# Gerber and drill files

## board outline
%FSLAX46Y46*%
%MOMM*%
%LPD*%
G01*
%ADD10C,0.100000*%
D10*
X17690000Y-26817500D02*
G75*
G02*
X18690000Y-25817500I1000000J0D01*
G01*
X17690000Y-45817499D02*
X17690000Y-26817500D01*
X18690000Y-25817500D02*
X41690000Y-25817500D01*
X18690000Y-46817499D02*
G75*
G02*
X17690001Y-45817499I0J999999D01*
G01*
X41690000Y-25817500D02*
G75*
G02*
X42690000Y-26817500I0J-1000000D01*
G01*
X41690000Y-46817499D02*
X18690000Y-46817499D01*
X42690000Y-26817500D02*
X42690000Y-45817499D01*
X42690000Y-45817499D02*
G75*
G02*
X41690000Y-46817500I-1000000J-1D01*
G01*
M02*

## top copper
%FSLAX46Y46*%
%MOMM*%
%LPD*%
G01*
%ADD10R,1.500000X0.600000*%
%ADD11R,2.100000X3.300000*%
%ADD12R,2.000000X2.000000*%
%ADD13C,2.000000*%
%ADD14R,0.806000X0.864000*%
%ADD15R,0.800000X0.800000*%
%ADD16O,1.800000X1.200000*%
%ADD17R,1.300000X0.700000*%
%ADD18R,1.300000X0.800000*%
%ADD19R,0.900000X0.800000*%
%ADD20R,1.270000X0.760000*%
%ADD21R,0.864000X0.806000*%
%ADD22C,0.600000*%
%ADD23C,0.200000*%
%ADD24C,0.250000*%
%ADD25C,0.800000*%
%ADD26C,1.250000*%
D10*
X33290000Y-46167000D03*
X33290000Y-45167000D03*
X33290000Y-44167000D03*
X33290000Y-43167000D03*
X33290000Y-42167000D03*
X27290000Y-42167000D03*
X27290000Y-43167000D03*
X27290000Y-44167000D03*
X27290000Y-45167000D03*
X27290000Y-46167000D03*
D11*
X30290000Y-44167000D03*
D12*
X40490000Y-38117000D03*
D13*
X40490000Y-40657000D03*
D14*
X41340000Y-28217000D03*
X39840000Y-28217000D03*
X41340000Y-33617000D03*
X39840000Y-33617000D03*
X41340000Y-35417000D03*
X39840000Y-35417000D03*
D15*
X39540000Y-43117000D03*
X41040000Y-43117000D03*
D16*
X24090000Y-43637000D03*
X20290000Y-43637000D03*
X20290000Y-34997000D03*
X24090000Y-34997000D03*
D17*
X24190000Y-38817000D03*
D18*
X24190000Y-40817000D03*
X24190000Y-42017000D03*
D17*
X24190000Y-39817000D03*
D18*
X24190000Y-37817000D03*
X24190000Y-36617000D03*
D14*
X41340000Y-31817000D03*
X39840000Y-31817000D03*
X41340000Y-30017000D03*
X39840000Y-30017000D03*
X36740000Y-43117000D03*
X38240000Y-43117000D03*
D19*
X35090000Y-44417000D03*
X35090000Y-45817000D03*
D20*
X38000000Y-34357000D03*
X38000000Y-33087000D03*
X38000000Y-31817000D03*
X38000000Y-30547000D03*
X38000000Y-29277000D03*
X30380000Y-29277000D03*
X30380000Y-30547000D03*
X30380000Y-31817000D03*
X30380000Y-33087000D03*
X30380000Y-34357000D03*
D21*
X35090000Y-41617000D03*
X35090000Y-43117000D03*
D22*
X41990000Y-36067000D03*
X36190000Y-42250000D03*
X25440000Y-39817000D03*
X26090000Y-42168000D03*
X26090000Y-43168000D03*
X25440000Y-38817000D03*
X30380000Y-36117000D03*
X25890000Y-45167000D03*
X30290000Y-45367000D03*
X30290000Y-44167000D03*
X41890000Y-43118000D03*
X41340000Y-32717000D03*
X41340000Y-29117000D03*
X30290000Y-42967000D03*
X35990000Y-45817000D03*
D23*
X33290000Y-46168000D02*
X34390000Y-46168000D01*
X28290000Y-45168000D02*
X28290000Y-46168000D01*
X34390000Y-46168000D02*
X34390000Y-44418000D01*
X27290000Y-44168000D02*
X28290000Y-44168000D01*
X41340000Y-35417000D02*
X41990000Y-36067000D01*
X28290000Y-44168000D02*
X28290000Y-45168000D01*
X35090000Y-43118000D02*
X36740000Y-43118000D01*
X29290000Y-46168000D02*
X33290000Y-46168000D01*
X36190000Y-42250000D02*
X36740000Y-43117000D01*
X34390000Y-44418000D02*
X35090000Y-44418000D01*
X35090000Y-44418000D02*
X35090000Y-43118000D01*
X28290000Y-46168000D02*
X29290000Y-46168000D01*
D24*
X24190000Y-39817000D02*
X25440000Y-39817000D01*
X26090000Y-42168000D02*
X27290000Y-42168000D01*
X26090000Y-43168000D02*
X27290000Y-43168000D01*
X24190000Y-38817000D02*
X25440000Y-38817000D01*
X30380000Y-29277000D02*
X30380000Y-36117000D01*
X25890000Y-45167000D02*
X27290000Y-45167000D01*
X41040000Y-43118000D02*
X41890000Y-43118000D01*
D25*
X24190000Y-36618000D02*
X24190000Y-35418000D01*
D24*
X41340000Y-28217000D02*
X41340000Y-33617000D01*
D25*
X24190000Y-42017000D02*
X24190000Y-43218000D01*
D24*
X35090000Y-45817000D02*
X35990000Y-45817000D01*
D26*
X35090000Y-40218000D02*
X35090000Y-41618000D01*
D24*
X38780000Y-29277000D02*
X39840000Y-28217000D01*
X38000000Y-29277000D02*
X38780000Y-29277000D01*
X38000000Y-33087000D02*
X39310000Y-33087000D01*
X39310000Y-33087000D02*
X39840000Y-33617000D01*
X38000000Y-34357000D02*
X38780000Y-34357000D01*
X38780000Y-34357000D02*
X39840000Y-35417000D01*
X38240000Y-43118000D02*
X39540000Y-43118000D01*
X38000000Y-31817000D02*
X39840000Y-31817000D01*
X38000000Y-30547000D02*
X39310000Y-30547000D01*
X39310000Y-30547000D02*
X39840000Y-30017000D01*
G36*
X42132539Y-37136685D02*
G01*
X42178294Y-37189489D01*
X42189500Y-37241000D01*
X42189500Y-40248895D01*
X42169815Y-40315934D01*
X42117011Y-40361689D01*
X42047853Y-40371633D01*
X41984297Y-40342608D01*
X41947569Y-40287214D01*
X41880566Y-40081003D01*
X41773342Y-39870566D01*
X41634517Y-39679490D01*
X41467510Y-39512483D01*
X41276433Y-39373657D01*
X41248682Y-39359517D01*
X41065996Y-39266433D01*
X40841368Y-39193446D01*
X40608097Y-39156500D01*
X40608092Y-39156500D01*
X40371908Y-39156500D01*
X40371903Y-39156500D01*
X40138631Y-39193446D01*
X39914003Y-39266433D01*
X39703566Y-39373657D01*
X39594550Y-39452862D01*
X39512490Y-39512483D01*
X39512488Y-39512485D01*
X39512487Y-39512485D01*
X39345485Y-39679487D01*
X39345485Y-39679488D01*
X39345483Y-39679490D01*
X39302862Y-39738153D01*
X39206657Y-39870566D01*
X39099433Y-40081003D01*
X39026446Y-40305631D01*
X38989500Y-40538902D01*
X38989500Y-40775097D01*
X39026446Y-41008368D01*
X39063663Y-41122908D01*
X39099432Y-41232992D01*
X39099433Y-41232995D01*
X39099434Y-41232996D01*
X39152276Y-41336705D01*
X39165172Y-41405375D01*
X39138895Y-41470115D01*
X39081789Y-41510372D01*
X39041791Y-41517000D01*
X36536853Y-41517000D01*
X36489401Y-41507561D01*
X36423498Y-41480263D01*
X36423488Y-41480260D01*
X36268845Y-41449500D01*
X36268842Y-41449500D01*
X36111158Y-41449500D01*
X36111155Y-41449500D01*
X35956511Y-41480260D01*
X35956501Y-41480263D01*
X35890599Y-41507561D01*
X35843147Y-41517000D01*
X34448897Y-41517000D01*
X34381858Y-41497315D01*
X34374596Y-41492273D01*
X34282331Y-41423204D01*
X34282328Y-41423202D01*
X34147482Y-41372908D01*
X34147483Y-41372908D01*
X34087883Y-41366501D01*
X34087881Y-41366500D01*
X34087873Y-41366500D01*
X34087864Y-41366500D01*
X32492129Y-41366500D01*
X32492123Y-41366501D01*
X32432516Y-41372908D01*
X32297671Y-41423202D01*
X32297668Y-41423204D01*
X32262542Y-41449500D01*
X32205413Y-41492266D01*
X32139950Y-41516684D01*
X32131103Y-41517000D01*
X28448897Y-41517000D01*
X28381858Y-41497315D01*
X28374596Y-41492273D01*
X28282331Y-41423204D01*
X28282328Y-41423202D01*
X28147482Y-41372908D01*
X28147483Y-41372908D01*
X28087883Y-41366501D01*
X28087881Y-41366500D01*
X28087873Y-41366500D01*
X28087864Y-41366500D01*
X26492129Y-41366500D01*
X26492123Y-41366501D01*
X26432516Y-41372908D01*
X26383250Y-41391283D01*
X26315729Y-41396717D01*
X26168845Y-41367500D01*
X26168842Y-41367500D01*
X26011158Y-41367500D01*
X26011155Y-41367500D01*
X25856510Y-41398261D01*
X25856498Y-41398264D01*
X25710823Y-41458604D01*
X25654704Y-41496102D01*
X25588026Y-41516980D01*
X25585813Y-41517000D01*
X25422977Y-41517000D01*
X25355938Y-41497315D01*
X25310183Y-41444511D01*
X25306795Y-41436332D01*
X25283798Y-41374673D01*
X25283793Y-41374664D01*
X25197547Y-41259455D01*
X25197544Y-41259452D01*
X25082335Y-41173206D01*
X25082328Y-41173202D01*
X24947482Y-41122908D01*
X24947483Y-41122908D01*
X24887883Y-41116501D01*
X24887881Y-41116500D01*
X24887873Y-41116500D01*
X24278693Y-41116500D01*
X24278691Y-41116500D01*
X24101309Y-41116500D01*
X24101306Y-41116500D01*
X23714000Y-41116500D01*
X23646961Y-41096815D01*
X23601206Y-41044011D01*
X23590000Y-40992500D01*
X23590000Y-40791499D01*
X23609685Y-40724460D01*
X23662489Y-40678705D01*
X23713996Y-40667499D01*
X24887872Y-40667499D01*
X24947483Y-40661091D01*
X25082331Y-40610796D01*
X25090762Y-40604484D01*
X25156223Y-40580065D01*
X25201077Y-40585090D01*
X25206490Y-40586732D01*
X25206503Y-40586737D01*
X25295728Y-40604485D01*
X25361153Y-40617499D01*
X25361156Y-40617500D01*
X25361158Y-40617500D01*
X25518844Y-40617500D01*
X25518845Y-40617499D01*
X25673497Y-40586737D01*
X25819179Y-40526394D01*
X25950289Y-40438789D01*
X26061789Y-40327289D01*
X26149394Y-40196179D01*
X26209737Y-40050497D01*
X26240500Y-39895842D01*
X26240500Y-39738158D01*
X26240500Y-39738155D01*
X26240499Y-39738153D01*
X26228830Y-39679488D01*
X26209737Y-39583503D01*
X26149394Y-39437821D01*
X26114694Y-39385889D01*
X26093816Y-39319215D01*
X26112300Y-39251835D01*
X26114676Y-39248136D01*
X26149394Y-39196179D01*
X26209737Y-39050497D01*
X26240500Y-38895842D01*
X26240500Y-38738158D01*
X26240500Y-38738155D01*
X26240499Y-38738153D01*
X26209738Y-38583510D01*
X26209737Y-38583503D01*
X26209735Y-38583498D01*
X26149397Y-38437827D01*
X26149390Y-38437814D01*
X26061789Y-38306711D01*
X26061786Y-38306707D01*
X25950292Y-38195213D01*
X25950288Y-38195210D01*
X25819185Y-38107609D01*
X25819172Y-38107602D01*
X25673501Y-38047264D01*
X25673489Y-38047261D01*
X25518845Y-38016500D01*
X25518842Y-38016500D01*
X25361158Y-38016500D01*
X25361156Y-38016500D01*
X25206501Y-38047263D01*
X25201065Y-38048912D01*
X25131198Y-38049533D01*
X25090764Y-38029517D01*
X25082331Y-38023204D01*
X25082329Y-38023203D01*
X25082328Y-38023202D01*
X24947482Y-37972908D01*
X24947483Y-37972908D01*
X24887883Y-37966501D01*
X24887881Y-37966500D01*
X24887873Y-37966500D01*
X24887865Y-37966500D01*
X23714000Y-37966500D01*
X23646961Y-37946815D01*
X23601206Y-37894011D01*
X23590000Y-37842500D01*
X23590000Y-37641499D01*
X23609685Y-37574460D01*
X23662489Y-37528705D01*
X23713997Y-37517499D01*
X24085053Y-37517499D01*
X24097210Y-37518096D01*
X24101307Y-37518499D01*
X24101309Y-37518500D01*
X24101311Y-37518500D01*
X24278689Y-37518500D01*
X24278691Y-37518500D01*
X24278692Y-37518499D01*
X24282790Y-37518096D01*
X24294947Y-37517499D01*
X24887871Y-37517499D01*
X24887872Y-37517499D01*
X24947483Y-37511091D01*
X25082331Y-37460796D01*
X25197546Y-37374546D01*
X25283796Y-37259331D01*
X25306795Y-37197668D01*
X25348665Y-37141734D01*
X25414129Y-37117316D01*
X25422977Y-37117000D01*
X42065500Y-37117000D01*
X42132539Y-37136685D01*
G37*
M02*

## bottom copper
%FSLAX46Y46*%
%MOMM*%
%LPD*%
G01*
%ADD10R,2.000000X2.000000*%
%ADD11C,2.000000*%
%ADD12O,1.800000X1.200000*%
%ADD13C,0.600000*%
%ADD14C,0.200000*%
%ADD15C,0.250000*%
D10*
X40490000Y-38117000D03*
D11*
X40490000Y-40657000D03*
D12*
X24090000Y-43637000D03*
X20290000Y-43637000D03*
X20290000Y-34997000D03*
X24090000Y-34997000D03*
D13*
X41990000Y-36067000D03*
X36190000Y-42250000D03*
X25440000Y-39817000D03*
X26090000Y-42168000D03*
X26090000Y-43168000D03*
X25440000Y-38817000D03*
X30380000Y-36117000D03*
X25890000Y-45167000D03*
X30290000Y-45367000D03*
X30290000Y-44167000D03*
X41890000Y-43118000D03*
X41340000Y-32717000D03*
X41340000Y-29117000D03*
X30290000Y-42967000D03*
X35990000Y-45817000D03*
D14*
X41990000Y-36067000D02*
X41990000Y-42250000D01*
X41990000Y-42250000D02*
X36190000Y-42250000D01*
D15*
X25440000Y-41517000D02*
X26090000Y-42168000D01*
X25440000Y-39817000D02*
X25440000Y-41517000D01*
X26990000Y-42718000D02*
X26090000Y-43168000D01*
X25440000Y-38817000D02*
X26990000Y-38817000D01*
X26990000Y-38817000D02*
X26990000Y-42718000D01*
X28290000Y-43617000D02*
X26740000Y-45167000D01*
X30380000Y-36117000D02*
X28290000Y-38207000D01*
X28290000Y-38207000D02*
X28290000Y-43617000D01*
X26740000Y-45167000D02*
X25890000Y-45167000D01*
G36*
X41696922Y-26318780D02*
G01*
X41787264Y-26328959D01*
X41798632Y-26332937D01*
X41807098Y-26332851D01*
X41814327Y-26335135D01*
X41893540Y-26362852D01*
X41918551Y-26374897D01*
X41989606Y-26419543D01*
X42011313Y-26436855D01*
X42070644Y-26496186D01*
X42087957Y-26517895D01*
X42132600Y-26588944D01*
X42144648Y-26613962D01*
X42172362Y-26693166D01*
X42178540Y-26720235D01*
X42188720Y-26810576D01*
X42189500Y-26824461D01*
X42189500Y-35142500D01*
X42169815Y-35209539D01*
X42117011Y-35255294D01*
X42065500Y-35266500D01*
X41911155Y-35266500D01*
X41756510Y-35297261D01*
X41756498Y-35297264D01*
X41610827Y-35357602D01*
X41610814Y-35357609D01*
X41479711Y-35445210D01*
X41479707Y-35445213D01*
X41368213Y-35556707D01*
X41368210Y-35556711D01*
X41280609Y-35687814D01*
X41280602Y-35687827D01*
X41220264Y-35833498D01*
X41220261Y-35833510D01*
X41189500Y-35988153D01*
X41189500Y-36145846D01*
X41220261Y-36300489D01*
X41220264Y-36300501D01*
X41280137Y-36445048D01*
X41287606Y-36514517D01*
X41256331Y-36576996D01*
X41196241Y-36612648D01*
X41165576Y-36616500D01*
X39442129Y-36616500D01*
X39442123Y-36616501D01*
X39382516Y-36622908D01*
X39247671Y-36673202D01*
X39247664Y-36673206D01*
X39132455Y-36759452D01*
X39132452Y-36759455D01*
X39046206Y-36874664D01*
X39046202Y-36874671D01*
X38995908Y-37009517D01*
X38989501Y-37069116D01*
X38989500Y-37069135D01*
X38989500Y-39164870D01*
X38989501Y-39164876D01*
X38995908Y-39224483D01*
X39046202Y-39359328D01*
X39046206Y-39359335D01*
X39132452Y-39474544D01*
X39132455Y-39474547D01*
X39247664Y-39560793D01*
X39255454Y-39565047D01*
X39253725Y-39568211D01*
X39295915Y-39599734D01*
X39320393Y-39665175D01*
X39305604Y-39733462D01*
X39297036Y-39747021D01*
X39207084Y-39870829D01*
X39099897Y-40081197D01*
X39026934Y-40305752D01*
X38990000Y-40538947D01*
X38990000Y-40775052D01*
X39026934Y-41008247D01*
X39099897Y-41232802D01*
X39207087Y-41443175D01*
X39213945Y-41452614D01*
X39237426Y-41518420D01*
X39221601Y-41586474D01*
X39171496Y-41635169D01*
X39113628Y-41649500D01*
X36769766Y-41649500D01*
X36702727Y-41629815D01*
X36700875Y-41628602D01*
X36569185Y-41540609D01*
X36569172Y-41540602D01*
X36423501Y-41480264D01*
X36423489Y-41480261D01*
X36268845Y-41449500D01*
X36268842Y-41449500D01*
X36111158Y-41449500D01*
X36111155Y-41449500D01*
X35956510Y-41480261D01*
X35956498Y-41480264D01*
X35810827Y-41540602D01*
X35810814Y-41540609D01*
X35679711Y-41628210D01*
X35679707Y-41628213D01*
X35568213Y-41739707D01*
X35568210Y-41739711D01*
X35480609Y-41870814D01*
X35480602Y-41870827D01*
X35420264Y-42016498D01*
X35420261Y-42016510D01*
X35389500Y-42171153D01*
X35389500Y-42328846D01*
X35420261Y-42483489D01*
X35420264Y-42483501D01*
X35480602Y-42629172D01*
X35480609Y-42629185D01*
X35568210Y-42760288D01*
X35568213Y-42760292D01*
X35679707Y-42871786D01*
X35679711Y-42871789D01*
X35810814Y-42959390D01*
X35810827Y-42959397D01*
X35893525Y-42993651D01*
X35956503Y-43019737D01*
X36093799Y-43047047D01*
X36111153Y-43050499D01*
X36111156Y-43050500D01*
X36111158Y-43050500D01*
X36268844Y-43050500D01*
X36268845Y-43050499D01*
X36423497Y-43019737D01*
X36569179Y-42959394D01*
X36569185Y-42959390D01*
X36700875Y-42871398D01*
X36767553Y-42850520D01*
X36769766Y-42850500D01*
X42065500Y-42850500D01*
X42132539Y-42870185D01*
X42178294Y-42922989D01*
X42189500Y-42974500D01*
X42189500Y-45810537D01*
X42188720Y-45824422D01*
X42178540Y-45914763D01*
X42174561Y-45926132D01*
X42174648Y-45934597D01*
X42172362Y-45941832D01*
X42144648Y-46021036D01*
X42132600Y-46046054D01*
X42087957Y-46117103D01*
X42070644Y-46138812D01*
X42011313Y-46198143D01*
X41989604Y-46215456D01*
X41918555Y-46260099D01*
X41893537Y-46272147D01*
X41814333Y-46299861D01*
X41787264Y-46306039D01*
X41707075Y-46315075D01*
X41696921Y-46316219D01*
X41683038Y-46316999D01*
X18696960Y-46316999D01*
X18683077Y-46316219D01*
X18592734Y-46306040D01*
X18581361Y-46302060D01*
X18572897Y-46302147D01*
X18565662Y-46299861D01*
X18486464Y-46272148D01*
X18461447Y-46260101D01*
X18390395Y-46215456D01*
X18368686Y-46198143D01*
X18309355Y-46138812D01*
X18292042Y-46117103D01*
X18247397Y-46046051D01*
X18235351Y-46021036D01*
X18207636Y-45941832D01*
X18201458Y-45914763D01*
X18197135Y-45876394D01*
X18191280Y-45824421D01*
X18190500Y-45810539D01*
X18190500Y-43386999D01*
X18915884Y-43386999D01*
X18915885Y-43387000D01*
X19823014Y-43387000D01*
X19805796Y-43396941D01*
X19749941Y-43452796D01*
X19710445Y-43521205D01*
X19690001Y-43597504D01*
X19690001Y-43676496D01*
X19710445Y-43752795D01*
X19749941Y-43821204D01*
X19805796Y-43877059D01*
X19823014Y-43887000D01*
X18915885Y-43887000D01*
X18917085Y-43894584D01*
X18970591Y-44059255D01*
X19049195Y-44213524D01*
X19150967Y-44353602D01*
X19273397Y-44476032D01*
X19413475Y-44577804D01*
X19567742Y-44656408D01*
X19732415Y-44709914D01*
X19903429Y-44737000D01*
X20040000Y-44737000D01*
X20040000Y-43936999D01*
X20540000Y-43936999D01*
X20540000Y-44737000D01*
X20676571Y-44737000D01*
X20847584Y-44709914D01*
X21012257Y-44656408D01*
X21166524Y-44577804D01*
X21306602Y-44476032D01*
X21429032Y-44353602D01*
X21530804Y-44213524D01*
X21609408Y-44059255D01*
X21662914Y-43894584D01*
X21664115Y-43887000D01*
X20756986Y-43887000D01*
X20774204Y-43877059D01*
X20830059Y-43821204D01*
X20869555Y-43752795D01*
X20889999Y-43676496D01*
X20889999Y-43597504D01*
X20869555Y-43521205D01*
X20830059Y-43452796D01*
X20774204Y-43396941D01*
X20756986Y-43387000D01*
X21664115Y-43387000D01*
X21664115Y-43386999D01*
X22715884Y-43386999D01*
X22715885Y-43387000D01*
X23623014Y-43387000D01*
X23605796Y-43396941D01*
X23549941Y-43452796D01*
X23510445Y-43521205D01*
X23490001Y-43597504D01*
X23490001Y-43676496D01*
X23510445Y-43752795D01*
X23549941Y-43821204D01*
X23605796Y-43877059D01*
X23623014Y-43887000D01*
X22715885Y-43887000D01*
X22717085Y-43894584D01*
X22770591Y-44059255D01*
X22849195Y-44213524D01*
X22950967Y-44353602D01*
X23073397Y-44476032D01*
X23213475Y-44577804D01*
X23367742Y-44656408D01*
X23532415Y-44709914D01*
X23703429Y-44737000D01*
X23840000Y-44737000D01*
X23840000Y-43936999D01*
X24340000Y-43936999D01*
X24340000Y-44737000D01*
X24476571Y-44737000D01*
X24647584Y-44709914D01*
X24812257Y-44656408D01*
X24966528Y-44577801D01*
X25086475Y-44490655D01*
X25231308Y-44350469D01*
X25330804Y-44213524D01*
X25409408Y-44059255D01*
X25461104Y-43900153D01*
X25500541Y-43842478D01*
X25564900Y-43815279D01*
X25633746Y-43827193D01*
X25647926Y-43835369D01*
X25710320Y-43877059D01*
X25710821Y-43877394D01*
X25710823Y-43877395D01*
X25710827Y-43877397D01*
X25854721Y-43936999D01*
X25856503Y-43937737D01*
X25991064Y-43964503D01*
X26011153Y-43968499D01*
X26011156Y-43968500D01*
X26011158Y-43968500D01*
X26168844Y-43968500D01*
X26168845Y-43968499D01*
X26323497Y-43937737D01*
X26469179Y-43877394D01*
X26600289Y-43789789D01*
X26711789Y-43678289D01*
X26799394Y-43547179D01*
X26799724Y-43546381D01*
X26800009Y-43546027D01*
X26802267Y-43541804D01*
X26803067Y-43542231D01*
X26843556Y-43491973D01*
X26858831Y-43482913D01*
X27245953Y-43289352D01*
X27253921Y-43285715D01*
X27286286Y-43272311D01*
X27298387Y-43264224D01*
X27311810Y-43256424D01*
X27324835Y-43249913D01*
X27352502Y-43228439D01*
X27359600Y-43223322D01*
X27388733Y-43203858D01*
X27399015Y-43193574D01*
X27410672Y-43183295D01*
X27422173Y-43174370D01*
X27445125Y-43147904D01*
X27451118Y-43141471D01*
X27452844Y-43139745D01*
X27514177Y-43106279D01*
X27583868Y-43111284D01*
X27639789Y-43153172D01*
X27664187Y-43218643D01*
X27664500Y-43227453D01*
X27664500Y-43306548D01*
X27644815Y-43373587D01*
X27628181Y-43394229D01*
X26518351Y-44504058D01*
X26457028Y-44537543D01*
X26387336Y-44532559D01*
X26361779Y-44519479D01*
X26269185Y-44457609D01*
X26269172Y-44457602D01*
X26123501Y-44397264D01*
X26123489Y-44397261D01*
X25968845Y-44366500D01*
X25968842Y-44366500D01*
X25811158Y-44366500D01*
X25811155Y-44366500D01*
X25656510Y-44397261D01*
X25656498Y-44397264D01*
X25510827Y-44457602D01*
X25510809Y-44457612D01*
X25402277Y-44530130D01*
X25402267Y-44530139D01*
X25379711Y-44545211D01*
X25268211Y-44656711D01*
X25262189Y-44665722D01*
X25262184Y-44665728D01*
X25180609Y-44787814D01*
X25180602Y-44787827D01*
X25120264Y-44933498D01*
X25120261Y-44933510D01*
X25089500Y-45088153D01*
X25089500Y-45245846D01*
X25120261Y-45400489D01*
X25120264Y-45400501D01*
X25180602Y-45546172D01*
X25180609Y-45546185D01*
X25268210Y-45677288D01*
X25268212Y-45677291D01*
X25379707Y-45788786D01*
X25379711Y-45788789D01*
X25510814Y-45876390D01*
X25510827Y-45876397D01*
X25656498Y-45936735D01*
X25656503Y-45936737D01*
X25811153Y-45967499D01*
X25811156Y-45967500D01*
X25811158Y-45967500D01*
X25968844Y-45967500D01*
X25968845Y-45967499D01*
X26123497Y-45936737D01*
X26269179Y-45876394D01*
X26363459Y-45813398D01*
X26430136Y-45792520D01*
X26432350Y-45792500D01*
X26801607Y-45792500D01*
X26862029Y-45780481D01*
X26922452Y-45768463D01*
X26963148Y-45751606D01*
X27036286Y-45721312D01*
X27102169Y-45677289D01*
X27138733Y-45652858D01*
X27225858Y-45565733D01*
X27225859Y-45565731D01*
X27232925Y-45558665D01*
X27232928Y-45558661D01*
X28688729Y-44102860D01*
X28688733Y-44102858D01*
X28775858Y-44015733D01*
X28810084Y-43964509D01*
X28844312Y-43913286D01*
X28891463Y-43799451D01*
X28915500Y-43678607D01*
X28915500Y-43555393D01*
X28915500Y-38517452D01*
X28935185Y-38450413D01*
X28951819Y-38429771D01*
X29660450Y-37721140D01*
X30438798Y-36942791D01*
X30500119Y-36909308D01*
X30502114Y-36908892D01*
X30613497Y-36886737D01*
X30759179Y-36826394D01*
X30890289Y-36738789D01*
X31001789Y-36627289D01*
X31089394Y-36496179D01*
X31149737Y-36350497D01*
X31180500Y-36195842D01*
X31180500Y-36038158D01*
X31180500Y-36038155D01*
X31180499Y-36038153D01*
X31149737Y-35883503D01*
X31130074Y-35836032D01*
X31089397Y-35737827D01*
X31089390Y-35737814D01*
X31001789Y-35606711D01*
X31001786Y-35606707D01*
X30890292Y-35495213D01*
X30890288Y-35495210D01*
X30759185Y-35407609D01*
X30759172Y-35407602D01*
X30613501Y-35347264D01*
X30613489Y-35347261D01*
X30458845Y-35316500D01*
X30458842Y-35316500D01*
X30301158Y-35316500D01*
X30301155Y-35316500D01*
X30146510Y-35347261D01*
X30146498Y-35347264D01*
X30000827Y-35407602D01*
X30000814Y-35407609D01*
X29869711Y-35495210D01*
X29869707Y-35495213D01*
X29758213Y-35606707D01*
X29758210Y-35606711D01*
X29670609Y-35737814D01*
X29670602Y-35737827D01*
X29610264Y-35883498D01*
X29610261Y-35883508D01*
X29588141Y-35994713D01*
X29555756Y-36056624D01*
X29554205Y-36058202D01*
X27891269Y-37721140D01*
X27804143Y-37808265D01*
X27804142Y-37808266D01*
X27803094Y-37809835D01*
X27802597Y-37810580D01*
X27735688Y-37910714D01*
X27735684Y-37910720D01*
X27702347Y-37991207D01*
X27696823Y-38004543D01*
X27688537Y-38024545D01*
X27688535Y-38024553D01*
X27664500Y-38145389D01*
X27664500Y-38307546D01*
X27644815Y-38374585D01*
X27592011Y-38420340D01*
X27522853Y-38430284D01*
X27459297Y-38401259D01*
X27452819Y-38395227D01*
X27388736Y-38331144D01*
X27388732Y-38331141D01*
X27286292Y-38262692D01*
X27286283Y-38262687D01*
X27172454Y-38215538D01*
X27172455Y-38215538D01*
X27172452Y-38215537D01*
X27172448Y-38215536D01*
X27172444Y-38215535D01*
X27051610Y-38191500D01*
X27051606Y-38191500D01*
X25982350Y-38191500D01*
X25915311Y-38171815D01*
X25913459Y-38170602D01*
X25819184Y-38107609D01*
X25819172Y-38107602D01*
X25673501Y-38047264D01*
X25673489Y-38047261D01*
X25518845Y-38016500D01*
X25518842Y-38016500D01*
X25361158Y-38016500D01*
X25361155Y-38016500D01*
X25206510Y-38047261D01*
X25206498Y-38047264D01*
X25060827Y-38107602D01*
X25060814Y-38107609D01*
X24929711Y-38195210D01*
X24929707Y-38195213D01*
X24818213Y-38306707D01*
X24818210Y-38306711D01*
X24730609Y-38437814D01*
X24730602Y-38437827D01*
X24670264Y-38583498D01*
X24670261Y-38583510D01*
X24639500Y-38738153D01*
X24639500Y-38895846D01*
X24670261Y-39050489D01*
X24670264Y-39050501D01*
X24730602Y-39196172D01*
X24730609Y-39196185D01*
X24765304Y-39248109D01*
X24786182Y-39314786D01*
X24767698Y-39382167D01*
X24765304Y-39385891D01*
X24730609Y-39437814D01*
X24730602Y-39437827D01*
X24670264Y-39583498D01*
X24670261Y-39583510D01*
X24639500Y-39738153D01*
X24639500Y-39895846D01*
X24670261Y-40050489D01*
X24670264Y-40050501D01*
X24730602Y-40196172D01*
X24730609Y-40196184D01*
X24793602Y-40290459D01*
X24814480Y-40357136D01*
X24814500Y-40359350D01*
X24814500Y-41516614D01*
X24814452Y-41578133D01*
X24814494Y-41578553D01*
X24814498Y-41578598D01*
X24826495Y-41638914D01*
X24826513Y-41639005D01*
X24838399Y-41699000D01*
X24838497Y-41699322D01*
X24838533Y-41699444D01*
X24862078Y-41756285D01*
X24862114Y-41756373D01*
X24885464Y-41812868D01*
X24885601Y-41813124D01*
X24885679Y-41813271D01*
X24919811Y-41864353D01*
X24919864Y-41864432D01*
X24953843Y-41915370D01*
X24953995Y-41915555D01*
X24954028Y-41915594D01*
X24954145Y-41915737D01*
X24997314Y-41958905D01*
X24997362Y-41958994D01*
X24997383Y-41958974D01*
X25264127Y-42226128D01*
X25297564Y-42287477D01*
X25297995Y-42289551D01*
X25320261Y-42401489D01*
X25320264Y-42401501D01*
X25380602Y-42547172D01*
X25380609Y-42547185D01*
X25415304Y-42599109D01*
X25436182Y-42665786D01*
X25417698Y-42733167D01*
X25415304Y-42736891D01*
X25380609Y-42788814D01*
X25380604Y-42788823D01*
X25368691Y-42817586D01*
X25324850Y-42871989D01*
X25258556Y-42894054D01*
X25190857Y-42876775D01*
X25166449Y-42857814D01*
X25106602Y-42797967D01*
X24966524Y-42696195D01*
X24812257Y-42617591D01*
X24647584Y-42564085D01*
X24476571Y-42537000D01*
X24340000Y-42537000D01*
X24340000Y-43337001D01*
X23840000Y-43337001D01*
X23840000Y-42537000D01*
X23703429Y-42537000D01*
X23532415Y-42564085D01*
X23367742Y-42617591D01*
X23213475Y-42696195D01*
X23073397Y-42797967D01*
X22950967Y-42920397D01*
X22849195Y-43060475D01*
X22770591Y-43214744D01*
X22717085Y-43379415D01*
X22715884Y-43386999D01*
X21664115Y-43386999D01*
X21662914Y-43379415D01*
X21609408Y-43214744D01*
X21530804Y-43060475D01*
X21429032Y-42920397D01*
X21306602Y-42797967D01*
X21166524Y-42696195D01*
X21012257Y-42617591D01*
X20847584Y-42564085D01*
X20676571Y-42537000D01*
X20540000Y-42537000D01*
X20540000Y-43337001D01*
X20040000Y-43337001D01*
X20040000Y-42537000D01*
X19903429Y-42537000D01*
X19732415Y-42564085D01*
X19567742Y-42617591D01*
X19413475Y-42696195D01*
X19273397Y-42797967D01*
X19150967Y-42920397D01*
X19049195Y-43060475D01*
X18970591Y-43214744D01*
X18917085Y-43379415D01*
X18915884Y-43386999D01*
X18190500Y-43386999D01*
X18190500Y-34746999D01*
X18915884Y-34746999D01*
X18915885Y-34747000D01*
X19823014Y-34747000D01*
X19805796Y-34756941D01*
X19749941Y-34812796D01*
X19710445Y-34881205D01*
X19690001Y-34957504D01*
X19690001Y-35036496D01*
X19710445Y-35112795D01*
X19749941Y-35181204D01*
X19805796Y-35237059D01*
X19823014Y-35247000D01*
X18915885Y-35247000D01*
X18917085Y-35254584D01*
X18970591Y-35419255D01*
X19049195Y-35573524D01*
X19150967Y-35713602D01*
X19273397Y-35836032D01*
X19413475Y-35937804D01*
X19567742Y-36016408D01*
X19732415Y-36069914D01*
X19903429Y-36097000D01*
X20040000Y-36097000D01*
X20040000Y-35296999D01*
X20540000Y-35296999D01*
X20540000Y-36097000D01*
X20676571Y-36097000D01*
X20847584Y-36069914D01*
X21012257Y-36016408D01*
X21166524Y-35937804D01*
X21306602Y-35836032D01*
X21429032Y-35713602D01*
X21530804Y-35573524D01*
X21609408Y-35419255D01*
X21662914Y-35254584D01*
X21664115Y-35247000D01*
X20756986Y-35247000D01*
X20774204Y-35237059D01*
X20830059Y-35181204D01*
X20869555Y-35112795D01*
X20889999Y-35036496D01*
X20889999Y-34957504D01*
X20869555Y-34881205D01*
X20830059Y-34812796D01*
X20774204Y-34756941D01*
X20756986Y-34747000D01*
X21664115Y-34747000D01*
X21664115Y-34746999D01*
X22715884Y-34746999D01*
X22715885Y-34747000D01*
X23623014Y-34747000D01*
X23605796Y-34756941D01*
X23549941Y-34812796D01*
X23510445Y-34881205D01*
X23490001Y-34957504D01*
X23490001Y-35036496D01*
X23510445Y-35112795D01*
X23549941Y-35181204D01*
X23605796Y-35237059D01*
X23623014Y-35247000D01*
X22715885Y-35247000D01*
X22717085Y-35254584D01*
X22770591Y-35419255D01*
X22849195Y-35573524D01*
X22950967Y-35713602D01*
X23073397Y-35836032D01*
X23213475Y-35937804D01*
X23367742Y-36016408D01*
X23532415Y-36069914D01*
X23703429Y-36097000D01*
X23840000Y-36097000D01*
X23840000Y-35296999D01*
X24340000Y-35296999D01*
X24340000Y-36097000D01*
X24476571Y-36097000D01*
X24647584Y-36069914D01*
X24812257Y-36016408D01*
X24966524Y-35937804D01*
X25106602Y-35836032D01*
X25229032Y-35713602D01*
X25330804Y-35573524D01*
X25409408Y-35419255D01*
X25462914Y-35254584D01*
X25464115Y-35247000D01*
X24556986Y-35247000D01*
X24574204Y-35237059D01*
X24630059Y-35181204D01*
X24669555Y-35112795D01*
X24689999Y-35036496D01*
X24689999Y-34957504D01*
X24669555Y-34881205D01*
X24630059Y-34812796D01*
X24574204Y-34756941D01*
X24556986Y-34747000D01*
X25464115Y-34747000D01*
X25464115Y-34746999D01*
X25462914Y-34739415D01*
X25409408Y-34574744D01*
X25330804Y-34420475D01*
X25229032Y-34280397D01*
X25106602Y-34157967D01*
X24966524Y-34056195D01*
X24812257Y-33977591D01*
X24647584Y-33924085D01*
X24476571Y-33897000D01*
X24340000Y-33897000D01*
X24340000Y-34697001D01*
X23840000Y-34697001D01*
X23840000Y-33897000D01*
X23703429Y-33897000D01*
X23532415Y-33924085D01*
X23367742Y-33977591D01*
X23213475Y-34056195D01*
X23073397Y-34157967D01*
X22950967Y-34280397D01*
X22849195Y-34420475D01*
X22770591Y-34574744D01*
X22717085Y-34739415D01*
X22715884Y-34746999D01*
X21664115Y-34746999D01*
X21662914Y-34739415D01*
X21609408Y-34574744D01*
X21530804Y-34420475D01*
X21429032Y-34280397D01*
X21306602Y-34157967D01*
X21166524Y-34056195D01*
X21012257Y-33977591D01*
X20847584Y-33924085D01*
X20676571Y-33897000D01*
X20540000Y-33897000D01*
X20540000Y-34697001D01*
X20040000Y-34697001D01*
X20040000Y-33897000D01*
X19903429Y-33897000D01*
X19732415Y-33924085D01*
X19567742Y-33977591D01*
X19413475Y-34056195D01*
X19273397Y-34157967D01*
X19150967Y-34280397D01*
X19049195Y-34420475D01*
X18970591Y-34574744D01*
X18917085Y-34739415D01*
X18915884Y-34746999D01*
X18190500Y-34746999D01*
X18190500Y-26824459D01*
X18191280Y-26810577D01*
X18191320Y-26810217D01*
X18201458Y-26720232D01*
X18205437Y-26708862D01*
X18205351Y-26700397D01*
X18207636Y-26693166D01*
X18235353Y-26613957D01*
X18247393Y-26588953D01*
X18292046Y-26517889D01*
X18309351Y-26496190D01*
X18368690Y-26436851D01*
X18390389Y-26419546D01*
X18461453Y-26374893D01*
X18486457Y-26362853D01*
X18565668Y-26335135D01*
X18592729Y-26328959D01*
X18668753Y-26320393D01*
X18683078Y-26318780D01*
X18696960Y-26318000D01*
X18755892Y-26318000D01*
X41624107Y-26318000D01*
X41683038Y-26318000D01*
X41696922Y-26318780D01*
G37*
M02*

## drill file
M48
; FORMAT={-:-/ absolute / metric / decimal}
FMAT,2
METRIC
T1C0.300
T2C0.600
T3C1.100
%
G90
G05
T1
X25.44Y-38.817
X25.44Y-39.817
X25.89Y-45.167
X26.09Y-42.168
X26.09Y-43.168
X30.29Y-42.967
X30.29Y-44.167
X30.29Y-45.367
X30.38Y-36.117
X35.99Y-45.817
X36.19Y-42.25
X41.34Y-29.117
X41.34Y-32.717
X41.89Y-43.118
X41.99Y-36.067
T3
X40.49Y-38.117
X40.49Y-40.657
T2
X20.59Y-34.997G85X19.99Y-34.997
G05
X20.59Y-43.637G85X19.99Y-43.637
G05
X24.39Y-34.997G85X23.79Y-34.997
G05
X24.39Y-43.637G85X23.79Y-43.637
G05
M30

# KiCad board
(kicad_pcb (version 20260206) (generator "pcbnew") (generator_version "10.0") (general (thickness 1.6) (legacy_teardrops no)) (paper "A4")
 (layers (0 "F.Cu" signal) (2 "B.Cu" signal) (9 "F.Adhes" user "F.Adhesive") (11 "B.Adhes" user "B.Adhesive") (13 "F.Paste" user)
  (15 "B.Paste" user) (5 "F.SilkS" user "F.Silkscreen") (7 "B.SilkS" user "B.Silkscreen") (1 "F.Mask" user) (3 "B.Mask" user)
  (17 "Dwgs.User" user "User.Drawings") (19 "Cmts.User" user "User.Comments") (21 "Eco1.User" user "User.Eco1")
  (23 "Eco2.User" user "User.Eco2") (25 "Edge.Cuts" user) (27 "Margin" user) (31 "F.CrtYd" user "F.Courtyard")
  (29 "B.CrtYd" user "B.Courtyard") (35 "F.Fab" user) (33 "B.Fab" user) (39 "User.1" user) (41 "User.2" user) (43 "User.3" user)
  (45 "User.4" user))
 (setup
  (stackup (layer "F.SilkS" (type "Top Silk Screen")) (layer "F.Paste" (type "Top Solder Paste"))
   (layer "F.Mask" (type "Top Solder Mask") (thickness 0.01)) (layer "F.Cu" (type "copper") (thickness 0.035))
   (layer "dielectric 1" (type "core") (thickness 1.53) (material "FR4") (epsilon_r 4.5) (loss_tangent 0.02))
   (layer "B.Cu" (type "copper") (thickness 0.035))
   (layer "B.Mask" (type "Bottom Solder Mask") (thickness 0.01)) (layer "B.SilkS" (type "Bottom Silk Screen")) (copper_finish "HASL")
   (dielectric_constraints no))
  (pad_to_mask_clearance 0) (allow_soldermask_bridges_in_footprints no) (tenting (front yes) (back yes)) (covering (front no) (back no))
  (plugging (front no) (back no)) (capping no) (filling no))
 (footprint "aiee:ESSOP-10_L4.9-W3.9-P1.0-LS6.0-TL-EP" (layer "F.Cu") (at 30.29 44.167 90)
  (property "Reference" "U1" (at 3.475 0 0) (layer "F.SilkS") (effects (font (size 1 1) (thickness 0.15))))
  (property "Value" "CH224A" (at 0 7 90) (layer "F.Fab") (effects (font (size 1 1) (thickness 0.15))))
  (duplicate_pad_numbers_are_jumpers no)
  (pad "1" smd rect (at -2 3 180) (size 1.5 0.6) (layers "F.Cu" "F.Mask" "F.Paste") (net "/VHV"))
  (pad "2" smd rect (at -1 3 180) (size 1.5 0.6) (layers "F.Cu" "F.Mask" "F.Paste") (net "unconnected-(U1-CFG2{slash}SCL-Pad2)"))
  (pad "3" smd rect (at 0 3 180) (size 1.5 0.6) (layers "F.Cu" "F.Mask" "F.Paste") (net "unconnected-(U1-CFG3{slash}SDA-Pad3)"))
  (pad "4" smd rect (at 1 3 180) (size 1.5 0.6) (layers "F.Cu" "F.Mask" "F.Paste") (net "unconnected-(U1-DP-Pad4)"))
  (pad "5" smd rect (at 2 3 180) (size 1.5 0.6) (layers "F.Cu" "F.Mask" "F.Paste") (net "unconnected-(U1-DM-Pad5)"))
  (pad "6" smd rect (at 2 -3 180) (size 1.5 0.6) (layers "F.Cu" "F.Mask" "F.Paste") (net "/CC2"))
  (pad "7" smd rect (at 1 -3 180) (size 1.5 0.6) (layers "F.Cu" "F.Mask" "F.Paste") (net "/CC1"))
  (pad "8" smd rect (at 0 -3 180) (size 1.5 0.6) (layers "F.Cu" "F.Mask" "F.Paste") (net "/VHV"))
  (pad "9" smd rect (at -1 -3 180) (size 1.5 0.6) (layers "F.Cu" "F.Mask" "F.Paste") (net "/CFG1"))
  (pad "10" smd rect (at -2 -3 180) (size 1.5 0.6) (layers "F.Cu" "F.Mask" "F.Paste") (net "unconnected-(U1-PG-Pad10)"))
  (pad "11" smd rect (at 0 0 270) (size 3.3 2.1) (layers "F.Cu" "F.Mask" "F.Paste") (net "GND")))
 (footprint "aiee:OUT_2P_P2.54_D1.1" (layer "F.Cu") (at 40.49 38.117)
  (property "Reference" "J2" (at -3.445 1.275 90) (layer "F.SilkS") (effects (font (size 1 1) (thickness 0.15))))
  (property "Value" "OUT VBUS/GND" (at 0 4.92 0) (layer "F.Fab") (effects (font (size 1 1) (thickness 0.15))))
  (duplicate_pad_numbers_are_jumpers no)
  (pad "1" thru_hole rect (at 0 0) (size 2 2) (drill 1.1) (layers "*.Cu" "*.Mask") (remove_unused_layers no) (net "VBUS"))
  (pad "2" thru_hole circle (at 0 2.54) (size 2 2) (drill 1.1) (layers "*.Cu" "*.Mask") (remove_unused_layers no) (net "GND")))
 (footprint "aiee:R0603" (layer "F.Cu") (at 40.59 28.217 180)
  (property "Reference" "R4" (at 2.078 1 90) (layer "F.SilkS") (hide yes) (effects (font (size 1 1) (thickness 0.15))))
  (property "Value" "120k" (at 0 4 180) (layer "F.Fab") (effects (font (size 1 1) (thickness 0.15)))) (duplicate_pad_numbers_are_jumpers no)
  (pad "1" smd rect (at -0.75 0 180) (size 0.806 0.864) (layers "F.Cu" "F.Mask" "F.Paste") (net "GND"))
  (pad "2" smd rect (at 0.75 0 180) (size 0.806 0.864) (layers "F.Cu" "F.Mask" "F.Paste") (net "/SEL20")))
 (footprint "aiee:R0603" (layer "F.Cu") (at 40.59 33.617 180)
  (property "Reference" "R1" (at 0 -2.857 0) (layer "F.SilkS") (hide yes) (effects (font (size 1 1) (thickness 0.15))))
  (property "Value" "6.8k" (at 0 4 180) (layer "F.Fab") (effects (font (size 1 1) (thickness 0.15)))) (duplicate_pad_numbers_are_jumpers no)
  (pad "1" smd rect (at -0.75 0 180) (size 0.806 0.864) (layers "F.Cu" "F.Mask" "F.Paste") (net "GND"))
  (pad "2" smd rect (at 0.75 0 180) (size 0.806 0.864) (layers "F.Cu" "F.Mask" "F.Paste") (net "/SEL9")))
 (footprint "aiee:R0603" (layer "F.Cu") (at 40.59 35.417 180)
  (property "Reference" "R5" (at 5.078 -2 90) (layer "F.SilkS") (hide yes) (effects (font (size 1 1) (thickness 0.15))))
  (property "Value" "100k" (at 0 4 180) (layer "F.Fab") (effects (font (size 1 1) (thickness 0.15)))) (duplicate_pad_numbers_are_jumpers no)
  (pad "1" smd rect (at -0.75 0 180) (size 0.806 0.864) (layers "F.Cu" "F.Mask" "F.Paste") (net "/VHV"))
  (pad "2" smd rect (at 0.75 0 180) (size 0.806 0.864) (layers "F.Cu" "F.Mask" "F.Paste") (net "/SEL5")))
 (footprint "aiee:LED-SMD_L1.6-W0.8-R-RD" (layer "F.Cu") (at 40.29 43.117 180)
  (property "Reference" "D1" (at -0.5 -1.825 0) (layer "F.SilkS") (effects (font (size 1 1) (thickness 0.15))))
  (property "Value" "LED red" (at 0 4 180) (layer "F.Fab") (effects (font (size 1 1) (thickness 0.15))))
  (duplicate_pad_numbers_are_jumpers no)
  (pad "1" smd rect (at 0.75 0 180) (size 0.8 0.8) (layers "F.Cu" "F.Mask" "F.Paste") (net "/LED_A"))
  (pad "2" smd rect (at -0.75 0 180) (size 0.8 0.8) (layers "F.Cu" "F.Mask" "F.Paste") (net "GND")))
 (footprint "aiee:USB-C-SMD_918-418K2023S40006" (layer "F.Cu") (at 22.24 39.317 -90)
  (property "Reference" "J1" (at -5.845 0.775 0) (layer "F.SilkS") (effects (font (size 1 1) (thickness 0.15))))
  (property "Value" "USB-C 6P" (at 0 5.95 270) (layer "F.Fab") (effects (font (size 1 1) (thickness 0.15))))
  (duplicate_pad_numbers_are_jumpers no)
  (pad "1" thru_hole oval (at 4.32 -1.85 270) (size 1.2 1.8) (drill oval 0.599998 1.199998) (layers "*.Cu" "*.Mask")
   (remove_unused_layers no) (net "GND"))
  (pad "2" thru_hole oval (at 4.32 1.95 270) (size 1.2 1.8) (drill oval 0.599998 1.199998) (layers "*.Cu" "*.Mask")
   (remove_unused_layers no) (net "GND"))
  (pad "3" thru_hole oval (at -4.32 1.95 270) (size 1.2 1.8) (drill oval 0.599998 1.199998) (layers "*.Cu" "*.Mask")
   (remove_unused_layers no) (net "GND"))
  (pad "4" thru_hole oval (at -4.32 -1.85 270) (size 1.2 1.8) (drill oval 0.599998 1.199998) (layers "*.Cu" "*.Mask")
   (remove_unused_layers no) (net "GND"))
  (pad "A5" smd rect (at -0.5 -1.95 270) (size 0.7 1.3) (layers "F.Cu" "F.Mask" "F.Paste") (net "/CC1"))
  (pad "A9" smd rect (at 1.5 -1.95 270) (size 0.8 1.3) (layers "F.Cu" "F.Mask" "F.Paste") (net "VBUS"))
  (pad "A12" smd rect (at 2.7 -1.95 270) (size 0.8 1.3) (layers "F.Cu" "F.Mask" "F.Paste") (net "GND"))
  (pad "B5" smd rect (at 0.5 -1.95 270) (size 0.7 1.3) (layers "F.Cu" "F.Mask" "F.Paste") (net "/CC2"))
  (pad "B9" smd rect (at -1.5 -1.95 270) (size 0.8 1.3) (layers "F.Cu" "F.Mask" "F.Paste") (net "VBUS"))
  (pad "B12" smd rect (at -2.7 -1.95 270) (size 0.8 1.3) (layers "F.Cu" "F.Mask" "F.Paste") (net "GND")))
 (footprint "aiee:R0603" (layer "F.Cu") (at 40.59 31.817 180)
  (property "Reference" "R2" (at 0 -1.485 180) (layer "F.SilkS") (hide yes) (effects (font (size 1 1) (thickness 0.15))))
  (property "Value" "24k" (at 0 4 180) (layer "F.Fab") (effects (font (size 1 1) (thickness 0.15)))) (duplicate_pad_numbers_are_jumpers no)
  (pad "1" smd rect (at -0.75 0 180) (size 0.806 0.864) (layers "F.Cu" "F.Mask" "F.Paste") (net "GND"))
  (pad "2" smd rect (at 0.75 0 180) (size 0.806 0.864) (layers "F.Cu" "F.Mask" "F.Paste") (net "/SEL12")))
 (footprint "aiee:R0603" (layer "F.Cu") (at 40.59 30.017 180)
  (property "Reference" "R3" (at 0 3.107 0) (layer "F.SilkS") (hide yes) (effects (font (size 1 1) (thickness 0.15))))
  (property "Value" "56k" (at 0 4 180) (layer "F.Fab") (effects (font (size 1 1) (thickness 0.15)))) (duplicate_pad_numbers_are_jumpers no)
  (pad "1" smd rect (at -0.75 0 180) (size 0.806 0.864) (layers "F.Cu" "F.Mask" "F.Paste") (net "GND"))
  (pad "2" smd rect (at 0.75 0 180) (size 0.806 0.864) (layers "F.Cu" "F.Mask" "F.Paste") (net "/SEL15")))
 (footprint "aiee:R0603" (layer "F.Cu") (at 37.49 43.117)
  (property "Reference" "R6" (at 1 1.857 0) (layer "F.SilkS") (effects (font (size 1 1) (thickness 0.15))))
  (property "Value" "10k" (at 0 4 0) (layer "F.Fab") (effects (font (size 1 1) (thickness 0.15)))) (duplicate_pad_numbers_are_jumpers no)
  (pad "1" smd rect (at -0.75 0) (size 0.806 0.864) (layers "F.Cu" "F.Mask" "F.Paste") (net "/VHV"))
  (pad "2" smd rect (at 0.75 0) (size 0.806 0.864) (layers "F.Cu" "F.Mask" "F.Paste") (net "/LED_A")))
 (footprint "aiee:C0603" (layer "F.Cu") (at 35.09 45.117 -90)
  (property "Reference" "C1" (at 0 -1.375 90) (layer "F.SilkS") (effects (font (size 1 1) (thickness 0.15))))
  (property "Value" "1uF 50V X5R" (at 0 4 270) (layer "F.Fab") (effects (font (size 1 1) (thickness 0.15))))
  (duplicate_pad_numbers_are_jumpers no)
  (pad "1" smd rect (at -0.7 0 270) (size 0.8 0.9) (layers "F.Cu" "F.Mask" "F.Paste") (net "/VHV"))
  (pad "2" smd rect (at 0.7 0 270) (size 0.8 0.9) (layers "F.Cu" "F.Mask" "F.Paste") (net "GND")))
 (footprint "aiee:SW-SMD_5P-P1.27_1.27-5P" (layer "F.Cu") (at 34.19 31.817 90)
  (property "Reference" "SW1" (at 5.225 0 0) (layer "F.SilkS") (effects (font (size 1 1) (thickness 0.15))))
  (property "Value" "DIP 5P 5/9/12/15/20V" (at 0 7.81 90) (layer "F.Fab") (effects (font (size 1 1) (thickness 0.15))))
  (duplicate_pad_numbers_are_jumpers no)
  (pad "1" smd rect (at -2.54 3.81 90) (size 0.76 1.27) (layers "F.Cu" "F.Mask" "F.Paste") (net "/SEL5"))
  (pad "2" smd rect (at -1.27 3.81 90) (size 0.76 1.27) (layers "F.Cu" "F.Mask" "F.Paste") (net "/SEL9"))
  (pad "3" smd rect (at 0 3.81 90) (size 0.76 1.27) (layers "F.Cu" "F.Mask" "F.Paste") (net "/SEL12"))
  (pad "4" smd rect (at 1.27 3.81 90) (size 0.76 1.27) (layers "F.Cu" "F.Mask" "F.Paste") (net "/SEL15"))
  (pad "5" smd rect (at 2.54 3.81 90) (size 0.76 1.27) (layers "F.Cu" "F.Mask" "F.Paste") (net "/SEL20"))
  (pad "6" smd rect (at 2.54 -3.81 90) (size 0.76 1.27) (layers "F.Cu" "F.Mask" "F.Paste") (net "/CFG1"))
  (pad "7" smd rect (at 1.27 -3.81 90) (size 0.76 1.27) (layers "F.Cu" "F.Mask" "F.Paste") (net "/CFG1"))
  (pad "8" smd rect (at 0 -3.81 90) (size 0.76 1.27) (layers "F.Cu" "F.Mask" "F.Paste") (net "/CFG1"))
  (pad "9" smd rect (at -1.27 -3.81 90) (size 0.76 1.27) (layers "F.Cu" "F.Mask" "F.Paste") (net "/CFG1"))
  (pad "10" smd rect (at -2.54 -3.81 90) (size 0.76 1.27) (layers "F.Cu" "F.Mask" "F.Paste") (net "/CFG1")))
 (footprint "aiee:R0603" (layer "F.Cu") (at 35.09 42.367 -90)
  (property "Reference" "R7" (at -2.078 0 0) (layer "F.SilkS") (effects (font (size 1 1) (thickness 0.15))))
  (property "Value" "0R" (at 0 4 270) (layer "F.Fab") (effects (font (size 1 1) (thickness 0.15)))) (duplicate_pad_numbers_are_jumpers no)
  (pad "1" smd rect (at -0.75 0 270) (size 0.806 0.864) (layers "F.Cu" "F.Mask" "F.Paste") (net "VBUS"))
  (pad "2" smd rect (at 0.75 0 270) (size 0.806 0.864) (layers "F.Cu" "F.Mask" "F.Paste") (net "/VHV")))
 (gr_arc (start 17.69 26.8175) (mid 17.982893 26.110393) (end 18.69 25.8175) (stroke (width 0.1) (type default)) (layer "Edge.Cuts"))
 (gr_line (start 17.69 45.817499) (end 17.69 26.8175) (stroke (width 0.1) (type default)) (layer "Edge.Cuts"))
 (gr_line (start 18.69 25.8175) (end 41.69 25.8175) (stroke (width 0.1) (type default)) (layer "Edge.Cuts"))
 (gr_arc (start 18.69 46.817499) (mid 17.982893 46.524606) (end 17.69 45.817499) (stroke (width 0.1) (type default)) (layer "Edge.Cuts"))
 (gr_arc (start 41.69 25.8175) (mid 42.397106 26.110393) (end 42.69 26.8175) (stroke (width 0.1) (type default)) (layer "Edge.Cuts"))
 (gr_line (start 41.69 46.817499) (end 18.69 46.817499) (stroke (width 0.1) (type default)) (layer "Edge.Cuts"))
 (gr_line (start 42.69 26.8175) (end 42.69 45.817499) (stroke (width 0.1) (type default)) (layer "Edge.Cuts"))
 (gr_arc (start 42.69 45.817499) (mid 42.397106 46.524606) (end 41.69 46.817499) (stroke (width 0.1) (type default)) (layer "Edge.Cuts"))
 (segment (start 33.29 46.168) (end 34.39 46.168) (width 0.2) (layer "F.Cu") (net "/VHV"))
 (segment (start 28.29 45.168) (end 28.29 46.168) (width 0.2) (layer "F.Cu") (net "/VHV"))
 (segment (start 34.39 46.168) (end 34.39 44.418) (width 0.2) (layer "F.Cu") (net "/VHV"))
 (segment (start 27.29 44.168) (end 28.29 44.168) (width 0.2) (layer "F.Cu") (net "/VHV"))
 (segment (start 41.34 35.417) (end 41.99 36.067) (width 0.2) (layer "F.Cu") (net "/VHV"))
 (segment (start 28.29 44.168) (end 28.29 45.168) (width 0.2) (layer "F.Cu") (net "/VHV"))
 (segment (start 35.09 43.118) (end 36.74 43.118) (width 0.2) (layer "F.Cu") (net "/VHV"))
 (segment (start 29.29 46.168) (end 33.29 46.168) (width 0.2) (layer "F.Cu") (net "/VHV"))
 (segment (start 36.19 42.25) (end 36.74 43.117) (width 0.2) (layer "F.Cu") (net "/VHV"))
 (segment (start 34.39 44.418) (end 35.09 44.418) (width 0.2) (layer "F.Cu") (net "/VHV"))
 (segment (start 35.09 44.418) (end 35.09 43.118) (width 0.2) (layer "F.Cu") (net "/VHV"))
 (segment (start 28.29 46.168) (end 29.29 46.168) (width 0.2) (layer "F.Cu") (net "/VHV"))
 (via (at 41.99 36.067) (size 0.6) (drill 0.3) (layers "F.Cu" "B.Cu") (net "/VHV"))
 (via (at 36.19 42.25) (size 0.6) (drill 0.3) (layers "F.Cu" "B.Cu") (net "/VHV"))
 (segment (start 41.99 36.067) (end 41.99 42.25) (width 0.2) (layer "B.Cu") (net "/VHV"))
 (segment (start 41.99 42.25) (end 36.19 42.25) (width 0.2) (layer "B.Cu") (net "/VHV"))
 (segment (start 24.19 39.817) (end 25.44 39.817) (width 0.25) (layer "F.Cu") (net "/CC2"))
 (segment (start 26.09 42.168) (end 27.29 42.168) (width 0.25) (layer "F.Cu") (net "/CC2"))
 (via (at 25.44 39.817) (size 0.6) (drill 0.3) (layers "F.Cu" "B.Cu") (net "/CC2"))
 (via (at 26.09 42.168) (size 0.6) (drill 0.3) (layers "F.Cu" "B.Cu") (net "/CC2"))
 (segment (start 25.44 41.517) (end 26.09 42.168) (width 0.25) (layer "B.Cu") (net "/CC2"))
 (segment (start 25.44 39.817) (end 25.44 41.517) (width 0.25) (layer "B.Cu") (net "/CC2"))
 (segment (start 26.09 43.168) (end 27.29 43.168) (width 0.25) (layer "F.Cu") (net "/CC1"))
 (segment (start 24.19 38.817) (end 25.44 38.817) (width 0.25) (layer "F.Cu") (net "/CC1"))
 (via (at 26.09 43.168) (size 0.6) (drill 0.3) (layers "F.Cu" "B.Cu") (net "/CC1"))
 (via (at 25.44 38.817) (size 0.6) (drill 0.3) (layers "F.Cu" "B.Cu") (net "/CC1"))
 (segment (start 26.99 42.718) (end 26.09 43.168) (width 0.25) (layer "B.Cu") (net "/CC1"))
 (segment (start 25.44 38.817) (end 26.99 38.817) (width 0.25) (layer "B.Cu") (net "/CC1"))
 (segment (start 26.99 38.817) (end 26.99 42.718) (width 0.25) (layer "B.Cu") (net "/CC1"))
 (segment (start 30.38 29.277) (end 30.38 36.117) (width 0.25) (layer "F.Cu") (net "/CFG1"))
 (segment (start 25.89 45.167) (end 27.29 45.167) (width 0.25) (layer "F.Cu") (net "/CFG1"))
 (via (at 30.38 36.117) (size 0.6) (drill 0.3) (layers "F.Cu" "B.Cu") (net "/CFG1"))
 (via (at 25.89 45.167) (size 0.6) (drill 0.3) (layers "F.Cu" "B.Cu") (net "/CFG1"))
 (segment (start 28.29 43.617) (end 26.74 45.167) (width 0.25) (layer "B.Cu") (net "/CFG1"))
 (segment (start 30.38 36.117) (end 28.29 38.207) (width 0.25) (layer "B.Cu") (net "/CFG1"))
 (segment (start 28.29 38.207) (end 28.29 43.617) (width 0.25) (layer "B.Cu") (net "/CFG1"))
 (segment (start 26.74 45.167) (end 25.89 45.167) (width 0.25) (layer "B.Cu") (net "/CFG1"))
 (segment (start 41.04 43.118) (end 41.89 43.118) (width 0.25) (layer "F.Cu") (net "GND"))
 (segment (start 24.19 36.618) (end 24.19 35.418) (width 0.8) (layer "F.Cu") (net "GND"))
 (segment (start 41.34 28.217) (end 41.34 33.617) (width 0.25) (layer "F.Cu") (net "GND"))
 (segment (start 24.19 42.017) (end 24.19 43.218) (width 0.8) (layer "F.Cu") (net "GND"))
 (segment (start 35.09 45.817) (end 35.99 45.817) (width 0.25) (layer "F.Cu") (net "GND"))
 (via (at 30.29 45.367) (size 0.6) (drill 0.3) (layers "F.Cu" "B.Cu") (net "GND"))
 (via (at 30.29 44.167) (size 0.6) (drill 0.3) (layers "F.Cu" "B.Cu") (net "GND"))
 (via (at 41.89 43.118) (size 0.6) (drill 0.3) (layers "F.Cu" "B.Cu") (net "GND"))
 (via (at 41.34 32.717) (size 0.6) (drill 0.3) (layers "F.Cu" "B.Cu") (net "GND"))
 (via (at 41.34 29.117) (size 0.6) (drill 0.3) (layers "F.Cu" "B.Cu") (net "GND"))
 (via (at 30.29 42.967) (size 0.6) (drill 0.3) (layers "F.Cu" "B.Cu") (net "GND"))
 (via (at 35.99 45.817) (size 0.6) (drill 0.3) (layers "F.Cu" "B.Cu") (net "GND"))
 (segment (start 35.09 40.218) (end 35.09 41.618) (width 1.25) (layer "F.Cu") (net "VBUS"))
 (segment (start 38.78 29.277) (end 39.84 28.217) (width 0.25) (layer "F.Cu") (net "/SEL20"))
 (segment (start 38 29.277) (end 38.78 29.277) (width 0.25) (layer "F.Cu") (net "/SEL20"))
 (segment (start 38 33.087) (end 39.31 33.087) (width 0.25) (layer "F.Cu") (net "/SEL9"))
 (segment (start 39.31 33.087) (end 39.84 33.617) (width 0.25) (layer "F.Cu") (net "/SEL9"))
 (segment (start 38 34.357) (end 38.78 34.357) (width 0.25) (layer "F.Cu") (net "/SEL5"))
 (segment (start 38.78 34.357) (end 39.84 35.417) (width 0.25) (layer "F.Cu") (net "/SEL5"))
 (segment (start 38.24 43.118) (end 39.54 43.118) (width 0.25) (layer "F.Cu") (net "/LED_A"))
 (segment (start 38 31.817) (end 39.84 31.817) (width 0.25) (layer "F.Cu") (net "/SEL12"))
 (segment (start 38 30.547) (end 39.31 30.547) (width 0.25) (layer "F.Cu") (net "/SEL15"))
 (segment (start 39.31 30.547) (end 39.84 30.017) (width 0.25) (layer "F.Cu") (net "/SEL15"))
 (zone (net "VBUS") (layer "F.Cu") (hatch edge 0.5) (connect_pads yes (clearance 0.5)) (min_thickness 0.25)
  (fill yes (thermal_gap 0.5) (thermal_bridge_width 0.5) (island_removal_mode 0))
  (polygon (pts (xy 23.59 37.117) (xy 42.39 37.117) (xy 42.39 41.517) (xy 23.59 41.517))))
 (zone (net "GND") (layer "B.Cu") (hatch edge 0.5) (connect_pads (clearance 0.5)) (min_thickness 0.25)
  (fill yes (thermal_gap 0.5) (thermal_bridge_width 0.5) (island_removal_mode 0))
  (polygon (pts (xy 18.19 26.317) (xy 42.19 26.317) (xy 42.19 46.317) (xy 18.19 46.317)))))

